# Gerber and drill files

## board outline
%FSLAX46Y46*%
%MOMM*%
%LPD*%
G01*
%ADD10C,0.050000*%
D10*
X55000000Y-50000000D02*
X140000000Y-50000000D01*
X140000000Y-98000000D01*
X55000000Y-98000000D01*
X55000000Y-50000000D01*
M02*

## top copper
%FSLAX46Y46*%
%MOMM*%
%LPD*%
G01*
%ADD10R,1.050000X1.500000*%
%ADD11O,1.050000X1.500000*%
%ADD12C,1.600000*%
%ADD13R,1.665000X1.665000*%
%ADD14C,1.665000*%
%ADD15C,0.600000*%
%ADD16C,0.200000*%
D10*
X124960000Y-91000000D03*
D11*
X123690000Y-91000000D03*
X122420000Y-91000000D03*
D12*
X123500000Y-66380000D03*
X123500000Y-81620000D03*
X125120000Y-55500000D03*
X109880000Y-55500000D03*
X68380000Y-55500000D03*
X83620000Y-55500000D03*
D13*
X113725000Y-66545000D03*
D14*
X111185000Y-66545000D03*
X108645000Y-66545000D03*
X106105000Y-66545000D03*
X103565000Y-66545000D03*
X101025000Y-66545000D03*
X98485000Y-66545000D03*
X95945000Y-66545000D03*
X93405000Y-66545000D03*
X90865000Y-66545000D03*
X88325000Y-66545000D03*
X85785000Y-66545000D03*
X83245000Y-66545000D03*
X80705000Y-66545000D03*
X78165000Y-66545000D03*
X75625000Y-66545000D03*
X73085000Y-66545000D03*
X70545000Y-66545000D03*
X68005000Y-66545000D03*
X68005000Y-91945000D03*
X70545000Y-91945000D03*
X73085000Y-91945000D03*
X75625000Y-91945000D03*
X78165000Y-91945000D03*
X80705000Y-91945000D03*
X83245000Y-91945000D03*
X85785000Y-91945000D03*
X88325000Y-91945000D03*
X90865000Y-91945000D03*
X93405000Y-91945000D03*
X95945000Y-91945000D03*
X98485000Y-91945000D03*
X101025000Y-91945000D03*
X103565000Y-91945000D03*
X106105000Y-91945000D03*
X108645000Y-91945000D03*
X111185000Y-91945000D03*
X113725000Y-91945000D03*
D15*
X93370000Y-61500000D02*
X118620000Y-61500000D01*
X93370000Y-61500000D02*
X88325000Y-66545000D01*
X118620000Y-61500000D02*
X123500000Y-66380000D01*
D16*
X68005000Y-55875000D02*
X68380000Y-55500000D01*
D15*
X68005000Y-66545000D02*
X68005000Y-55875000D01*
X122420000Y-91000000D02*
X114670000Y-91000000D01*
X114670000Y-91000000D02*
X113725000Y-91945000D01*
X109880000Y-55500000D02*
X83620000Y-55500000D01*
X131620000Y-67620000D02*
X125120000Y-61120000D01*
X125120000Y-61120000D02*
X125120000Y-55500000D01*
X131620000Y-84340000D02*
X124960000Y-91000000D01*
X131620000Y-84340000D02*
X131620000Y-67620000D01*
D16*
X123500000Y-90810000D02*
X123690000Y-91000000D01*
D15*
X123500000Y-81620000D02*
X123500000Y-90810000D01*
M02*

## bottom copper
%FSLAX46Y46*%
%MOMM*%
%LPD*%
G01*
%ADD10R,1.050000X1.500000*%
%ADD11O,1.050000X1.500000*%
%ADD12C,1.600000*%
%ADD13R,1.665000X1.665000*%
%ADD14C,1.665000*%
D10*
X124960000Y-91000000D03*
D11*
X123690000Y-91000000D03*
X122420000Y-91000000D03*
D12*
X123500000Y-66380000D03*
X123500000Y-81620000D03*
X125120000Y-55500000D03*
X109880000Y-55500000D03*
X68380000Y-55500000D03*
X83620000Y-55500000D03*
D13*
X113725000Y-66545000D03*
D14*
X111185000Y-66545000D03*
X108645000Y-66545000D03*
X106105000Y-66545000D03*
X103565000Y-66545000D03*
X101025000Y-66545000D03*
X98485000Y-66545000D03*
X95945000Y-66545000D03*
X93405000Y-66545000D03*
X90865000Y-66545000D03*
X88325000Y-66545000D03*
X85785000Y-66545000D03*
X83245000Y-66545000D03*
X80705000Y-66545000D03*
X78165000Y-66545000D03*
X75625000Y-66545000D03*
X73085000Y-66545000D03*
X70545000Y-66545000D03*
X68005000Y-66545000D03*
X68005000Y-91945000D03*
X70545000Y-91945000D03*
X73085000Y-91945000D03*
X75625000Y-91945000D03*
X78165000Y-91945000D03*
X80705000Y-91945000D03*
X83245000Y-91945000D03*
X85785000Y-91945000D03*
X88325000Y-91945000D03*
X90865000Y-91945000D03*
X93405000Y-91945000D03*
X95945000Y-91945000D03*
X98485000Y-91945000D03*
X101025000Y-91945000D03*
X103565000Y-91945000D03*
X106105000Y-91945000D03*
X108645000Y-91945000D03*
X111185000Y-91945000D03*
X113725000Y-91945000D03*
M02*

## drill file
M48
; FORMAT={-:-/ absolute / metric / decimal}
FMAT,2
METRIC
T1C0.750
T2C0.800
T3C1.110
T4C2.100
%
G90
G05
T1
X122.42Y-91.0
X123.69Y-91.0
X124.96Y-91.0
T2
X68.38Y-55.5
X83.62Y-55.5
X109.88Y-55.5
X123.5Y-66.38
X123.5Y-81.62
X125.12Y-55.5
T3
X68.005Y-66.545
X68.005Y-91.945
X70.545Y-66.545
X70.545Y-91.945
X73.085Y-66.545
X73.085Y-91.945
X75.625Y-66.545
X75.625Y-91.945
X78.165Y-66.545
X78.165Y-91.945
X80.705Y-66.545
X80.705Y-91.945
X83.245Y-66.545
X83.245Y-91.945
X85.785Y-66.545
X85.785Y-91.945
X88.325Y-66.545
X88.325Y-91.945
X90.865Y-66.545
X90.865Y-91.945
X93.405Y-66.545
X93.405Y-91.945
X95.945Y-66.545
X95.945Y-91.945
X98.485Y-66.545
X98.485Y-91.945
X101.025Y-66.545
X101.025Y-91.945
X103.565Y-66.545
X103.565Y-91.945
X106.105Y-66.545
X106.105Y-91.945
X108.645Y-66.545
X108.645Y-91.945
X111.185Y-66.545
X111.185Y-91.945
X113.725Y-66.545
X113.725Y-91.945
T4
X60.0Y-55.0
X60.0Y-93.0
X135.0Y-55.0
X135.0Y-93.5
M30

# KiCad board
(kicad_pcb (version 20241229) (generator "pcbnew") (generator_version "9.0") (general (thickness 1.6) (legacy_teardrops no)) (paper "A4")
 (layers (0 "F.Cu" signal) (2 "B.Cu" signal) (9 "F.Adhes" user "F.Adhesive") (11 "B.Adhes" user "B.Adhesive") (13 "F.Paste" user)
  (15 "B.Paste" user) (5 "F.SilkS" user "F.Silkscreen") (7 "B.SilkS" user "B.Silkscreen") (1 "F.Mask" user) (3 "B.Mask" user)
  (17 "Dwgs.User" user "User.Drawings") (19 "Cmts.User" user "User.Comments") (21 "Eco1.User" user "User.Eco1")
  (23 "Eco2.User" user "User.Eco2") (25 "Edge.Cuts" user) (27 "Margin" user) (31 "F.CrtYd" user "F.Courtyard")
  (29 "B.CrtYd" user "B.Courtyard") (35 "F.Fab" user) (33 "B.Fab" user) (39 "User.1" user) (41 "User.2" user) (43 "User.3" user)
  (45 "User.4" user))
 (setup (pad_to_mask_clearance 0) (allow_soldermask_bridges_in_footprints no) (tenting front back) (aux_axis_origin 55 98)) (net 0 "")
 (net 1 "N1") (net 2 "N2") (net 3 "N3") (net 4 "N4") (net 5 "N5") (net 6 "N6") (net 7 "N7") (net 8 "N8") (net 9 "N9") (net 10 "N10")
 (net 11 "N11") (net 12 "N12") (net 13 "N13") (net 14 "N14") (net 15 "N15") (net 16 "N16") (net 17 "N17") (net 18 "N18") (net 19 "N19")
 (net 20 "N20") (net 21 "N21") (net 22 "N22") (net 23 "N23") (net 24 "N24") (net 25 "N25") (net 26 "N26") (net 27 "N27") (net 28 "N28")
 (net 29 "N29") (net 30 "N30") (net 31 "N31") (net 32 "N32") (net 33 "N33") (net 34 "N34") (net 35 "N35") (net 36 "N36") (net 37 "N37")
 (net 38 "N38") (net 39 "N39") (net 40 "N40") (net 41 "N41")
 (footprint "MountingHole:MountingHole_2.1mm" (layer "F.Cu") (at 135 93.5)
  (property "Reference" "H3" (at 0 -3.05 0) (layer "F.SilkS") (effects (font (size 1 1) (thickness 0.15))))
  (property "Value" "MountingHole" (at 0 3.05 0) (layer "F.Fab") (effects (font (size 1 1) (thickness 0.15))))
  (pad "" np_thru_hole circle (at 0 0) (size 2.1 2.1) (drill 2.1) (layers "*.Cu" "*.Mask")))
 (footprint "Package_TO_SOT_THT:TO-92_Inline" (layer "F.Cu") (at 124.96 91 180)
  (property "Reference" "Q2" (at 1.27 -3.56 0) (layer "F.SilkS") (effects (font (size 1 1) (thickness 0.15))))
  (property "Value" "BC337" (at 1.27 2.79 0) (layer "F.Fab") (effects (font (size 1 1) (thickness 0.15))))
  (pad "1" thru_hole rect (at 0 0 180) (size 1.05 1.5) (drill 0.75) (layers "*.Cu" "*.Mask") (remove_unused_layers no) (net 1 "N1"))
  (pad "2" thru_hole oval (at 1.27 0 180) (size 1.05 1.5) (drill 0.75) (layers "*.Cu" "*.Mask") (remove_unused_layers no) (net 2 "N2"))
  (pad "3" thru_hole oval (at 2.54 0 180) (size 1.05 1.5) (drill 0.75) (layers "*.Cu" "*.Mask") (remove_unused_layers no) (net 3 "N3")))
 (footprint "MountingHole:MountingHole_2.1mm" (layer "F.Cu") (at 60 93)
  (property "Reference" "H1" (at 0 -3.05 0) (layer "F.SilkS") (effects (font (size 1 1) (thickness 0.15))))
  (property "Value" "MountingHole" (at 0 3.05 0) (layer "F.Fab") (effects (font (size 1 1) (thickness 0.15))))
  (pad "" np_thru_hole circle (at 0 0) (size 2.1 2.1) (drill 2.1) (layers "*.Cu" "*.Mask")))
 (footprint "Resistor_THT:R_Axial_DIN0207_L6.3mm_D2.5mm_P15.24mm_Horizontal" (layer "F.Cu") (at 123.5 66.38 -90)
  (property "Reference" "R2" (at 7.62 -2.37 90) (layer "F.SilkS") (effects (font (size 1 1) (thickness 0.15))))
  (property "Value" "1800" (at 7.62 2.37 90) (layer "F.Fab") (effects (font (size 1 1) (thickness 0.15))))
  (pad "1" thru_hole circle (at 0 0 270) (size 1.6 1.6) (drill 0.8) (layers "*.Cu" "*.Mask") (remove_unused_layers no) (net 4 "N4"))
  (pad "2" thru_hole circle (at 15.24 0 270) (size 1.6 1.6) (drill 0.8) (layers "*.Cu" "*.Mask") (remove_unused_layers no) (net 2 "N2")))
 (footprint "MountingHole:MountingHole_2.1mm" (layer "F.Cu") (at 60 55)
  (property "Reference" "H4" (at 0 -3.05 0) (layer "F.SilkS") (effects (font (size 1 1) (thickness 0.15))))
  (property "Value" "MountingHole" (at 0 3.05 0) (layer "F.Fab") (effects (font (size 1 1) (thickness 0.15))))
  (pad "" np_thru_hole circle (at 0 0) (size 2.1 2.1) (drill 2.1) (layers "*.Cu" "*.Mask")))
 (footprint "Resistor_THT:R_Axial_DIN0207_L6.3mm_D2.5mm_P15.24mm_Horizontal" (layer "F.Cu") (at 125.12 55.5 180)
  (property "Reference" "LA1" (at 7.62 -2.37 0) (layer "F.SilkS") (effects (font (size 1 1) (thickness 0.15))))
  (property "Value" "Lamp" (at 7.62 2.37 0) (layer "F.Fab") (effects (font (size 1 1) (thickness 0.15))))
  (pad "1" thru_hole circle (at 0 0 180) (size 1.6 1.6) (drill 0.8) (layers "*.Cu" "*.Mask") (remove_unused_layers no) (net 1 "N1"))
  (pad "2" thru_hole circle (at 15.24 0 180) (size 1.6 1.6) (drill 0.8) (layers "*.Cu" "*.Mask") (remove_unused_layers no) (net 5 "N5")))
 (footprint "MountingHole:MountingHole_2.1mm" (layer "F.Cu") (at 135 55)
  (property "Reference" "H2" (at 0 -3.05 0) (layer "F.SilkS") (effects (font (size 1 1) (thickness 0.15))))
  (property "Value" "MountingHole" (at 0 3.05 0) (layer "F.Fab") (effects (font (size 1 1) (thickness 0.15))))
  (pad "" np_thru_hole circle (at 0 0) (size 2.1 2.1) (drill 2.1) (layers "*.Cu" "*.Mask")))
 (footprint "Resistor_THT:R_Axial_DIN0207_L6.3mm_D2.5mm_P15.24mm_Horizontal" (layer "F.Cu") (at 68.38 55.5)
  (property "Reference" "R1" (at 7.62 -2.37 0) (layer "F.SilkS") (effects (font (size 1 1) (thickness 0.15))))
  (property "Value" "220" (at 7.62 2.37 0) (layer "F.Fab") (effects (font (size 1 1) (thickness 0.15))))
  (pad "1" thru_hole circle (at 0 0) (size 1.6 1.6) (drill 0.8) (layers "*.Cu" "*.Mask") (remove_unused_layers no) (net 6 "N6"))
  (pad "2" thru_hole circle (at 15.24 0) (size 1.6 1.6) (drill 0.8) (layers "*.Cu" "*.Mask") (remove_unused_layers no) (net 5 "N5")))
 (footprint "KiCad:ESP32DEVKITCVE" (layer "F.Cu") (at 113.725 66.545 -90)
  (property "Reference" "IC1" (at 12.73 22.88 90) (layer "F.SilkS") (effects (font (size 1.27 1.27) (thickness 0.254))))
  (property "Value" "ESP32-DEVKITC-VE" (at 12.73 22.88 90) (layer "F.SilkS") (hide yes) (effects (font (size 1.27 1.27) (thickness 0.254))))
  (pad "1" thru_hole rect (at 0 0 270) (size 1.665 1.665) (drill 1.11) (layers "*.Cu" "*.Mask") (remove_unused_layers no) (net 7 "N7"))
  (pad "2" thru_hole circle (at 0 2.54 270) (size 1.665 1.665) (drill 1.11) (layers "*.Cu" "*.Mask") (remove_unused_layers no) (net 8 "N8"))
  (pad "3" thru_hole circle (at 0 5.08 270) (size 1.665 1.665) (drill 1.11) (layers "*.Cu" "*.Mask") (remove_unused_layers no) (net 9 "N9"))
  (pad "4" thru_hole circle (at 0 7.62 270) (size 1.665 1.665) (drill 1.11) (layers "*.Cu" "*.Mask") (remove_unused_layers no)
   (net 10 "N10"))
  (pad "5" thru_hole circle (at 0 10.16 270) (size 1.665 1.665) (drill 1.11) (layers "*.Cu" "*.Mask") (remove_unused_layers no)
   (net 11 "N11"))
  (pad "6" thru_hole circle (at 0 12.7 270) (size 1.665 1.665) (drill 1.11) (layers "*.Cu" "*.Mask") (remove_unused_layers no)
   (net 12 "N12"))
  (pad "7" thru_hole circle (at 0 15.24 270) (size 1.665 1.665) (drill 1.11) (layers "*.Cu" "*.Mask") (remove_unused_layers no)
   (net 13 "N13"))
  (pad "8" thru_hole circle (at 0 17.78 270) (size 1.665 1.665) (drill 1.11) (layers "*.Cu" "*.Mask") (remove_unused_layers no)
   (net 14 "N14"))
  (pad "9" thru_hole circle (at 0 20.32 270) (size 1.665 1.665) (drill 1.11) (layers "*.Cu" "*.Mask") (remove_unused_layers no)
   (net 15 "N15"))
  (pad "10" thru_hole circle (at 0 22.86 270) (size 1.665 1.665) (drill 1.11) (layers "*.Cu" "*.Mask") (remove_unused_layers no)
   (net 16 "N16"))
  (pad "11" thru_hole circle (at 0 25.4 270) (size 1.665 1.665) (drill 1.11) (layers "*.Cu" "*.Mask") (remove_unused_layers no) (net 4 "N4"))
  (pad "12" thru_hole circle (at 0 27.94 270) (size 1.665 1.665) (drill 1.11) (layers "*.Cu" "*.Mask") (remove_unused_layers no)
   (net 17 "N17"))
  (pad "13" thru_hole circle (at 0 30.48 270) (size 1.665 1.665) (drill 1.11) (layers "*.Cu" "*.Mask") (remove_unused_layers no)
   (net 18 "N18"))
  (pad "14" thru_hole circle (at 0 33.02 270) (size 1.665 1.665) (drill 1.11) (layers "*.Cu" "*.Mask") (remove_unused_layers no)
   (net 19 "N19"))
  (pad "15" thru_hole circle (at 0 35.56 270) (size 1.665 1.665) (drill 1.11) (layers "*.Cu" "*.Mask") (remove_unused_layers no)
   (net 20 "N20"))
  (pad "16" thru_hole circle (at 0 38.1 270) (size 1.665 1.665) (drill 1.11) (layers "*.Cu" "*.Mask") (remove_unused_layers no)
   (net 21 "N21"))
  (pad "17" thru_hole circle (at 0 40.64 270) (size 1.665 1.665) (drill 1.11) (layers "*.Cu" "*.Mask") (remove_unused_layers no)
   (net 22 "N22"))
  (pad "18" thru_hole circle (at 0 43.18 270) (size 1.665 1.665) (drill 1.11) (layers "*.Cu" "*.Mask") (remove_unused_layers no)
   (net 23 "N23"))
  (pad "19" thru_hole circle (at 0 45.72 270) (size 1.665 1.665) (drill 1.11) (layers "*.Cu" "*.Mask") (remove_unused_layers no)
   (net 6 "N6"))
  (pad "20" thru_hole circle (at 25.4 45.72 270) (size 1.665 1.665) (drill 1.11) (layers "*.Cu" "*.Mask") (remove_unused_layers no)
   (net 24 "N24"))
  (pad "21" thru_hole circle (at 25.4 43.18 270) (size 1.665 1.665) (drill 1.11) (layers "*.Cu" "*.Mask") (remove_unused_layers no)
   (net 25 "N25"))
  (pad "22" thru_hole circle (at 25.4 40.64 270) (size 1.665 1.665) (drill 1.11) (layers "*.Cu" "*.Mask") (remove_unused_layers no)
   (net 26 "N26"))
  (pad "23" thru_hole circle (at 25.4 38.1 270) (size 1.665 1.665) (drill 1.11) (layers "*.Cu" "*.Mask") (remove_unused_layers no)
   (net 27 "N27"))
  (pad "24" thru_hole circle (at 25.4 35.56 270) (size 1.665 1.665) (drill 1.11) (layers "*.Cu" "*.Mask") (remove_unused_layers no)
   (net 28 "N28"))
  (pad "25" thru_hole circle (at 25.4 33.02 270) (size 1.665 1.665) (drill 1.11) (layers "*.Cu" "*.Mask") (remove_unused_layers no)
   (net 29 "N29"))
  (pad "26" thru_hole circle (at 25.4 30.48 270) (size 1.665 1.665) (drill 1.11) (layers "*.Cu" "*.Mask") (remove_unused_layers no)
   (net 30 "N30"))
  (pad "27" thru_hole circle (at 25.4 27.94 270) (size 1.665 1.665) (drill 1.11) (layers "*.Cu" "*.Mask") (remove_unused_layers no)
   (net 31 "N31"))
  (pad "28" thru_hole circle (at 25.4 25.4 270) (size 1.665 1.665) (drill 1.11) (layers "*.Cu" "*.Mask") (remove_unused_layers no)
   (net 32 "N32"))
  (pad "29" thru_hole circle (at 25.4 22.86 270) (size 1.665 1.665) (drill 1.11) (layers "*.Cu" "*.Mask") (remove_unused_layers no)
   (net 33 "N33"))
  (pad "30" thru_hole circle (at 25.4 20.32 270) (size 1.665 1.665) (drill 1.11) (layers "*.Cu" "*.Mask") (remove_unused_layers no)
   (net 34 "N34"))
  (pad "31" thru_hole circle (at 25.4 17.78 270) (size 1.665 1.665) (drill 1.11) (layers "*.Cu" "*.Mask") (remove_unused_layers no)
   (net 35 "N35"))
  (pad "32" thru_hole circle (at 25.4 15.24 270) (size 1.665 1.665) (drill 1.11) (layers "*.Cu" "*.Mask") (remove_unused_layers no)
   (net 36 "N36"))
  (pad "33" thru_hole circle (at 25.4 12.7 270) (size 1.665 1.665) (drill 1.11) (layers "*.Cu" "*.Mask") (remove_unused_layers no)
   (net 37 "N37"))
  (pad "34" thru_hole circle (at 25.4 10.16 270) (size 1.665 1.665) (drill 1.11) (layers "*.Cu" "*.Mask") (remove_unused_layers no)
   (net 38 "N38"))
  (pad "35" thru_hole circle (at 25.4 7.62 270) (size 1.665 1.665) (drill 1.11) (layers "*.Cu" "*.Mask") (remove_unused_layers no)
   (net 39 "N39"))
  (pad "36" thru_hole circle (at 25.4 5.08 270) (size 1.665 1.665) (drill 1.11) (layers "*.Cu" "*.Mask") (remove_unused_layers no)
   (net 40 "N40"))
  (pad "37" thru_hole circle (at 25.4 2.54 270) (size 1.665 1.665) (drill 1.11) (layers "*.Cu" "*.Mask") (remove_unused_layers no)
   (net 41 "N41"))
  (pad "38" thru_hole circle (at 25.4 0 270) (size 1.665 1.665) (drill 1.11) (layers "*.Cu" "*.Mask") (remove_unused_layers no) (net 3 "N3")))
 (gr_rect (start 55 50) (end 140 98) (stroke (width 0.05) (type default)) (fill no) (layer "Edge.Cuts"))
 (segment (start 93.37 61.5) (end 118.62 61.5) (width 0.6) (layer "F.Cu") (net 4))
 (segment (start 93.37 61.5) (end 88.325 66.545) (width 0.6) (layer "F.Cu") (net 4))
 (segment (start 118.62 61.5) (end 123.5 66.38) (width 0.6) (layer "F.Cu") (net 4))
 (segment (start 68.005 55.875) (end 68.38 55.5) (width 0.2) (layer "F.Cu") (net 6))
 (segment (start 68.005 66.545) (end 68.005 55.875) (width 0.6) (layer "F.Cu") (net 6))
 (segment (start 122.42 91) (end 114.67 91) (width 0.6) (layer "F.Cu") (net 3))
 (segment (start 114.67 91) (end 113.725 91.945) (width 0.6) (layer "F.Cu") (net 3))
 (segment (start 109.88 55.5) (end 83.62 55.5) (width 0.6) (layer "F.Cu") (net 5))
 (segment (start 131.62 67.62) (end 125.12 61.12) (width 0.6) (layer "F.Cu") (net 1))
 (segment (start 125.12 61.12) (end 125.12 55.5) (width 0.6) (layer "F.Cu") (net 1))
 (segment (start 131.62 84.34) (end 124.96 91) (width 0.6) (layer "F.Cu") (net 1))
 (segment (start 131.62 84.34) (end 131.62 67.62) (width 0.6) (layer "F.Cu") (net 1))
 (segment (start 123.5 90.81) (end 123.69 91) (width 0.2) (layer "F.Cu") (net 2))
 (segment (start 123.5 81.62) (end 123.5 90.81) (width 0.6) (layer "F.Cu") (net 2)))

